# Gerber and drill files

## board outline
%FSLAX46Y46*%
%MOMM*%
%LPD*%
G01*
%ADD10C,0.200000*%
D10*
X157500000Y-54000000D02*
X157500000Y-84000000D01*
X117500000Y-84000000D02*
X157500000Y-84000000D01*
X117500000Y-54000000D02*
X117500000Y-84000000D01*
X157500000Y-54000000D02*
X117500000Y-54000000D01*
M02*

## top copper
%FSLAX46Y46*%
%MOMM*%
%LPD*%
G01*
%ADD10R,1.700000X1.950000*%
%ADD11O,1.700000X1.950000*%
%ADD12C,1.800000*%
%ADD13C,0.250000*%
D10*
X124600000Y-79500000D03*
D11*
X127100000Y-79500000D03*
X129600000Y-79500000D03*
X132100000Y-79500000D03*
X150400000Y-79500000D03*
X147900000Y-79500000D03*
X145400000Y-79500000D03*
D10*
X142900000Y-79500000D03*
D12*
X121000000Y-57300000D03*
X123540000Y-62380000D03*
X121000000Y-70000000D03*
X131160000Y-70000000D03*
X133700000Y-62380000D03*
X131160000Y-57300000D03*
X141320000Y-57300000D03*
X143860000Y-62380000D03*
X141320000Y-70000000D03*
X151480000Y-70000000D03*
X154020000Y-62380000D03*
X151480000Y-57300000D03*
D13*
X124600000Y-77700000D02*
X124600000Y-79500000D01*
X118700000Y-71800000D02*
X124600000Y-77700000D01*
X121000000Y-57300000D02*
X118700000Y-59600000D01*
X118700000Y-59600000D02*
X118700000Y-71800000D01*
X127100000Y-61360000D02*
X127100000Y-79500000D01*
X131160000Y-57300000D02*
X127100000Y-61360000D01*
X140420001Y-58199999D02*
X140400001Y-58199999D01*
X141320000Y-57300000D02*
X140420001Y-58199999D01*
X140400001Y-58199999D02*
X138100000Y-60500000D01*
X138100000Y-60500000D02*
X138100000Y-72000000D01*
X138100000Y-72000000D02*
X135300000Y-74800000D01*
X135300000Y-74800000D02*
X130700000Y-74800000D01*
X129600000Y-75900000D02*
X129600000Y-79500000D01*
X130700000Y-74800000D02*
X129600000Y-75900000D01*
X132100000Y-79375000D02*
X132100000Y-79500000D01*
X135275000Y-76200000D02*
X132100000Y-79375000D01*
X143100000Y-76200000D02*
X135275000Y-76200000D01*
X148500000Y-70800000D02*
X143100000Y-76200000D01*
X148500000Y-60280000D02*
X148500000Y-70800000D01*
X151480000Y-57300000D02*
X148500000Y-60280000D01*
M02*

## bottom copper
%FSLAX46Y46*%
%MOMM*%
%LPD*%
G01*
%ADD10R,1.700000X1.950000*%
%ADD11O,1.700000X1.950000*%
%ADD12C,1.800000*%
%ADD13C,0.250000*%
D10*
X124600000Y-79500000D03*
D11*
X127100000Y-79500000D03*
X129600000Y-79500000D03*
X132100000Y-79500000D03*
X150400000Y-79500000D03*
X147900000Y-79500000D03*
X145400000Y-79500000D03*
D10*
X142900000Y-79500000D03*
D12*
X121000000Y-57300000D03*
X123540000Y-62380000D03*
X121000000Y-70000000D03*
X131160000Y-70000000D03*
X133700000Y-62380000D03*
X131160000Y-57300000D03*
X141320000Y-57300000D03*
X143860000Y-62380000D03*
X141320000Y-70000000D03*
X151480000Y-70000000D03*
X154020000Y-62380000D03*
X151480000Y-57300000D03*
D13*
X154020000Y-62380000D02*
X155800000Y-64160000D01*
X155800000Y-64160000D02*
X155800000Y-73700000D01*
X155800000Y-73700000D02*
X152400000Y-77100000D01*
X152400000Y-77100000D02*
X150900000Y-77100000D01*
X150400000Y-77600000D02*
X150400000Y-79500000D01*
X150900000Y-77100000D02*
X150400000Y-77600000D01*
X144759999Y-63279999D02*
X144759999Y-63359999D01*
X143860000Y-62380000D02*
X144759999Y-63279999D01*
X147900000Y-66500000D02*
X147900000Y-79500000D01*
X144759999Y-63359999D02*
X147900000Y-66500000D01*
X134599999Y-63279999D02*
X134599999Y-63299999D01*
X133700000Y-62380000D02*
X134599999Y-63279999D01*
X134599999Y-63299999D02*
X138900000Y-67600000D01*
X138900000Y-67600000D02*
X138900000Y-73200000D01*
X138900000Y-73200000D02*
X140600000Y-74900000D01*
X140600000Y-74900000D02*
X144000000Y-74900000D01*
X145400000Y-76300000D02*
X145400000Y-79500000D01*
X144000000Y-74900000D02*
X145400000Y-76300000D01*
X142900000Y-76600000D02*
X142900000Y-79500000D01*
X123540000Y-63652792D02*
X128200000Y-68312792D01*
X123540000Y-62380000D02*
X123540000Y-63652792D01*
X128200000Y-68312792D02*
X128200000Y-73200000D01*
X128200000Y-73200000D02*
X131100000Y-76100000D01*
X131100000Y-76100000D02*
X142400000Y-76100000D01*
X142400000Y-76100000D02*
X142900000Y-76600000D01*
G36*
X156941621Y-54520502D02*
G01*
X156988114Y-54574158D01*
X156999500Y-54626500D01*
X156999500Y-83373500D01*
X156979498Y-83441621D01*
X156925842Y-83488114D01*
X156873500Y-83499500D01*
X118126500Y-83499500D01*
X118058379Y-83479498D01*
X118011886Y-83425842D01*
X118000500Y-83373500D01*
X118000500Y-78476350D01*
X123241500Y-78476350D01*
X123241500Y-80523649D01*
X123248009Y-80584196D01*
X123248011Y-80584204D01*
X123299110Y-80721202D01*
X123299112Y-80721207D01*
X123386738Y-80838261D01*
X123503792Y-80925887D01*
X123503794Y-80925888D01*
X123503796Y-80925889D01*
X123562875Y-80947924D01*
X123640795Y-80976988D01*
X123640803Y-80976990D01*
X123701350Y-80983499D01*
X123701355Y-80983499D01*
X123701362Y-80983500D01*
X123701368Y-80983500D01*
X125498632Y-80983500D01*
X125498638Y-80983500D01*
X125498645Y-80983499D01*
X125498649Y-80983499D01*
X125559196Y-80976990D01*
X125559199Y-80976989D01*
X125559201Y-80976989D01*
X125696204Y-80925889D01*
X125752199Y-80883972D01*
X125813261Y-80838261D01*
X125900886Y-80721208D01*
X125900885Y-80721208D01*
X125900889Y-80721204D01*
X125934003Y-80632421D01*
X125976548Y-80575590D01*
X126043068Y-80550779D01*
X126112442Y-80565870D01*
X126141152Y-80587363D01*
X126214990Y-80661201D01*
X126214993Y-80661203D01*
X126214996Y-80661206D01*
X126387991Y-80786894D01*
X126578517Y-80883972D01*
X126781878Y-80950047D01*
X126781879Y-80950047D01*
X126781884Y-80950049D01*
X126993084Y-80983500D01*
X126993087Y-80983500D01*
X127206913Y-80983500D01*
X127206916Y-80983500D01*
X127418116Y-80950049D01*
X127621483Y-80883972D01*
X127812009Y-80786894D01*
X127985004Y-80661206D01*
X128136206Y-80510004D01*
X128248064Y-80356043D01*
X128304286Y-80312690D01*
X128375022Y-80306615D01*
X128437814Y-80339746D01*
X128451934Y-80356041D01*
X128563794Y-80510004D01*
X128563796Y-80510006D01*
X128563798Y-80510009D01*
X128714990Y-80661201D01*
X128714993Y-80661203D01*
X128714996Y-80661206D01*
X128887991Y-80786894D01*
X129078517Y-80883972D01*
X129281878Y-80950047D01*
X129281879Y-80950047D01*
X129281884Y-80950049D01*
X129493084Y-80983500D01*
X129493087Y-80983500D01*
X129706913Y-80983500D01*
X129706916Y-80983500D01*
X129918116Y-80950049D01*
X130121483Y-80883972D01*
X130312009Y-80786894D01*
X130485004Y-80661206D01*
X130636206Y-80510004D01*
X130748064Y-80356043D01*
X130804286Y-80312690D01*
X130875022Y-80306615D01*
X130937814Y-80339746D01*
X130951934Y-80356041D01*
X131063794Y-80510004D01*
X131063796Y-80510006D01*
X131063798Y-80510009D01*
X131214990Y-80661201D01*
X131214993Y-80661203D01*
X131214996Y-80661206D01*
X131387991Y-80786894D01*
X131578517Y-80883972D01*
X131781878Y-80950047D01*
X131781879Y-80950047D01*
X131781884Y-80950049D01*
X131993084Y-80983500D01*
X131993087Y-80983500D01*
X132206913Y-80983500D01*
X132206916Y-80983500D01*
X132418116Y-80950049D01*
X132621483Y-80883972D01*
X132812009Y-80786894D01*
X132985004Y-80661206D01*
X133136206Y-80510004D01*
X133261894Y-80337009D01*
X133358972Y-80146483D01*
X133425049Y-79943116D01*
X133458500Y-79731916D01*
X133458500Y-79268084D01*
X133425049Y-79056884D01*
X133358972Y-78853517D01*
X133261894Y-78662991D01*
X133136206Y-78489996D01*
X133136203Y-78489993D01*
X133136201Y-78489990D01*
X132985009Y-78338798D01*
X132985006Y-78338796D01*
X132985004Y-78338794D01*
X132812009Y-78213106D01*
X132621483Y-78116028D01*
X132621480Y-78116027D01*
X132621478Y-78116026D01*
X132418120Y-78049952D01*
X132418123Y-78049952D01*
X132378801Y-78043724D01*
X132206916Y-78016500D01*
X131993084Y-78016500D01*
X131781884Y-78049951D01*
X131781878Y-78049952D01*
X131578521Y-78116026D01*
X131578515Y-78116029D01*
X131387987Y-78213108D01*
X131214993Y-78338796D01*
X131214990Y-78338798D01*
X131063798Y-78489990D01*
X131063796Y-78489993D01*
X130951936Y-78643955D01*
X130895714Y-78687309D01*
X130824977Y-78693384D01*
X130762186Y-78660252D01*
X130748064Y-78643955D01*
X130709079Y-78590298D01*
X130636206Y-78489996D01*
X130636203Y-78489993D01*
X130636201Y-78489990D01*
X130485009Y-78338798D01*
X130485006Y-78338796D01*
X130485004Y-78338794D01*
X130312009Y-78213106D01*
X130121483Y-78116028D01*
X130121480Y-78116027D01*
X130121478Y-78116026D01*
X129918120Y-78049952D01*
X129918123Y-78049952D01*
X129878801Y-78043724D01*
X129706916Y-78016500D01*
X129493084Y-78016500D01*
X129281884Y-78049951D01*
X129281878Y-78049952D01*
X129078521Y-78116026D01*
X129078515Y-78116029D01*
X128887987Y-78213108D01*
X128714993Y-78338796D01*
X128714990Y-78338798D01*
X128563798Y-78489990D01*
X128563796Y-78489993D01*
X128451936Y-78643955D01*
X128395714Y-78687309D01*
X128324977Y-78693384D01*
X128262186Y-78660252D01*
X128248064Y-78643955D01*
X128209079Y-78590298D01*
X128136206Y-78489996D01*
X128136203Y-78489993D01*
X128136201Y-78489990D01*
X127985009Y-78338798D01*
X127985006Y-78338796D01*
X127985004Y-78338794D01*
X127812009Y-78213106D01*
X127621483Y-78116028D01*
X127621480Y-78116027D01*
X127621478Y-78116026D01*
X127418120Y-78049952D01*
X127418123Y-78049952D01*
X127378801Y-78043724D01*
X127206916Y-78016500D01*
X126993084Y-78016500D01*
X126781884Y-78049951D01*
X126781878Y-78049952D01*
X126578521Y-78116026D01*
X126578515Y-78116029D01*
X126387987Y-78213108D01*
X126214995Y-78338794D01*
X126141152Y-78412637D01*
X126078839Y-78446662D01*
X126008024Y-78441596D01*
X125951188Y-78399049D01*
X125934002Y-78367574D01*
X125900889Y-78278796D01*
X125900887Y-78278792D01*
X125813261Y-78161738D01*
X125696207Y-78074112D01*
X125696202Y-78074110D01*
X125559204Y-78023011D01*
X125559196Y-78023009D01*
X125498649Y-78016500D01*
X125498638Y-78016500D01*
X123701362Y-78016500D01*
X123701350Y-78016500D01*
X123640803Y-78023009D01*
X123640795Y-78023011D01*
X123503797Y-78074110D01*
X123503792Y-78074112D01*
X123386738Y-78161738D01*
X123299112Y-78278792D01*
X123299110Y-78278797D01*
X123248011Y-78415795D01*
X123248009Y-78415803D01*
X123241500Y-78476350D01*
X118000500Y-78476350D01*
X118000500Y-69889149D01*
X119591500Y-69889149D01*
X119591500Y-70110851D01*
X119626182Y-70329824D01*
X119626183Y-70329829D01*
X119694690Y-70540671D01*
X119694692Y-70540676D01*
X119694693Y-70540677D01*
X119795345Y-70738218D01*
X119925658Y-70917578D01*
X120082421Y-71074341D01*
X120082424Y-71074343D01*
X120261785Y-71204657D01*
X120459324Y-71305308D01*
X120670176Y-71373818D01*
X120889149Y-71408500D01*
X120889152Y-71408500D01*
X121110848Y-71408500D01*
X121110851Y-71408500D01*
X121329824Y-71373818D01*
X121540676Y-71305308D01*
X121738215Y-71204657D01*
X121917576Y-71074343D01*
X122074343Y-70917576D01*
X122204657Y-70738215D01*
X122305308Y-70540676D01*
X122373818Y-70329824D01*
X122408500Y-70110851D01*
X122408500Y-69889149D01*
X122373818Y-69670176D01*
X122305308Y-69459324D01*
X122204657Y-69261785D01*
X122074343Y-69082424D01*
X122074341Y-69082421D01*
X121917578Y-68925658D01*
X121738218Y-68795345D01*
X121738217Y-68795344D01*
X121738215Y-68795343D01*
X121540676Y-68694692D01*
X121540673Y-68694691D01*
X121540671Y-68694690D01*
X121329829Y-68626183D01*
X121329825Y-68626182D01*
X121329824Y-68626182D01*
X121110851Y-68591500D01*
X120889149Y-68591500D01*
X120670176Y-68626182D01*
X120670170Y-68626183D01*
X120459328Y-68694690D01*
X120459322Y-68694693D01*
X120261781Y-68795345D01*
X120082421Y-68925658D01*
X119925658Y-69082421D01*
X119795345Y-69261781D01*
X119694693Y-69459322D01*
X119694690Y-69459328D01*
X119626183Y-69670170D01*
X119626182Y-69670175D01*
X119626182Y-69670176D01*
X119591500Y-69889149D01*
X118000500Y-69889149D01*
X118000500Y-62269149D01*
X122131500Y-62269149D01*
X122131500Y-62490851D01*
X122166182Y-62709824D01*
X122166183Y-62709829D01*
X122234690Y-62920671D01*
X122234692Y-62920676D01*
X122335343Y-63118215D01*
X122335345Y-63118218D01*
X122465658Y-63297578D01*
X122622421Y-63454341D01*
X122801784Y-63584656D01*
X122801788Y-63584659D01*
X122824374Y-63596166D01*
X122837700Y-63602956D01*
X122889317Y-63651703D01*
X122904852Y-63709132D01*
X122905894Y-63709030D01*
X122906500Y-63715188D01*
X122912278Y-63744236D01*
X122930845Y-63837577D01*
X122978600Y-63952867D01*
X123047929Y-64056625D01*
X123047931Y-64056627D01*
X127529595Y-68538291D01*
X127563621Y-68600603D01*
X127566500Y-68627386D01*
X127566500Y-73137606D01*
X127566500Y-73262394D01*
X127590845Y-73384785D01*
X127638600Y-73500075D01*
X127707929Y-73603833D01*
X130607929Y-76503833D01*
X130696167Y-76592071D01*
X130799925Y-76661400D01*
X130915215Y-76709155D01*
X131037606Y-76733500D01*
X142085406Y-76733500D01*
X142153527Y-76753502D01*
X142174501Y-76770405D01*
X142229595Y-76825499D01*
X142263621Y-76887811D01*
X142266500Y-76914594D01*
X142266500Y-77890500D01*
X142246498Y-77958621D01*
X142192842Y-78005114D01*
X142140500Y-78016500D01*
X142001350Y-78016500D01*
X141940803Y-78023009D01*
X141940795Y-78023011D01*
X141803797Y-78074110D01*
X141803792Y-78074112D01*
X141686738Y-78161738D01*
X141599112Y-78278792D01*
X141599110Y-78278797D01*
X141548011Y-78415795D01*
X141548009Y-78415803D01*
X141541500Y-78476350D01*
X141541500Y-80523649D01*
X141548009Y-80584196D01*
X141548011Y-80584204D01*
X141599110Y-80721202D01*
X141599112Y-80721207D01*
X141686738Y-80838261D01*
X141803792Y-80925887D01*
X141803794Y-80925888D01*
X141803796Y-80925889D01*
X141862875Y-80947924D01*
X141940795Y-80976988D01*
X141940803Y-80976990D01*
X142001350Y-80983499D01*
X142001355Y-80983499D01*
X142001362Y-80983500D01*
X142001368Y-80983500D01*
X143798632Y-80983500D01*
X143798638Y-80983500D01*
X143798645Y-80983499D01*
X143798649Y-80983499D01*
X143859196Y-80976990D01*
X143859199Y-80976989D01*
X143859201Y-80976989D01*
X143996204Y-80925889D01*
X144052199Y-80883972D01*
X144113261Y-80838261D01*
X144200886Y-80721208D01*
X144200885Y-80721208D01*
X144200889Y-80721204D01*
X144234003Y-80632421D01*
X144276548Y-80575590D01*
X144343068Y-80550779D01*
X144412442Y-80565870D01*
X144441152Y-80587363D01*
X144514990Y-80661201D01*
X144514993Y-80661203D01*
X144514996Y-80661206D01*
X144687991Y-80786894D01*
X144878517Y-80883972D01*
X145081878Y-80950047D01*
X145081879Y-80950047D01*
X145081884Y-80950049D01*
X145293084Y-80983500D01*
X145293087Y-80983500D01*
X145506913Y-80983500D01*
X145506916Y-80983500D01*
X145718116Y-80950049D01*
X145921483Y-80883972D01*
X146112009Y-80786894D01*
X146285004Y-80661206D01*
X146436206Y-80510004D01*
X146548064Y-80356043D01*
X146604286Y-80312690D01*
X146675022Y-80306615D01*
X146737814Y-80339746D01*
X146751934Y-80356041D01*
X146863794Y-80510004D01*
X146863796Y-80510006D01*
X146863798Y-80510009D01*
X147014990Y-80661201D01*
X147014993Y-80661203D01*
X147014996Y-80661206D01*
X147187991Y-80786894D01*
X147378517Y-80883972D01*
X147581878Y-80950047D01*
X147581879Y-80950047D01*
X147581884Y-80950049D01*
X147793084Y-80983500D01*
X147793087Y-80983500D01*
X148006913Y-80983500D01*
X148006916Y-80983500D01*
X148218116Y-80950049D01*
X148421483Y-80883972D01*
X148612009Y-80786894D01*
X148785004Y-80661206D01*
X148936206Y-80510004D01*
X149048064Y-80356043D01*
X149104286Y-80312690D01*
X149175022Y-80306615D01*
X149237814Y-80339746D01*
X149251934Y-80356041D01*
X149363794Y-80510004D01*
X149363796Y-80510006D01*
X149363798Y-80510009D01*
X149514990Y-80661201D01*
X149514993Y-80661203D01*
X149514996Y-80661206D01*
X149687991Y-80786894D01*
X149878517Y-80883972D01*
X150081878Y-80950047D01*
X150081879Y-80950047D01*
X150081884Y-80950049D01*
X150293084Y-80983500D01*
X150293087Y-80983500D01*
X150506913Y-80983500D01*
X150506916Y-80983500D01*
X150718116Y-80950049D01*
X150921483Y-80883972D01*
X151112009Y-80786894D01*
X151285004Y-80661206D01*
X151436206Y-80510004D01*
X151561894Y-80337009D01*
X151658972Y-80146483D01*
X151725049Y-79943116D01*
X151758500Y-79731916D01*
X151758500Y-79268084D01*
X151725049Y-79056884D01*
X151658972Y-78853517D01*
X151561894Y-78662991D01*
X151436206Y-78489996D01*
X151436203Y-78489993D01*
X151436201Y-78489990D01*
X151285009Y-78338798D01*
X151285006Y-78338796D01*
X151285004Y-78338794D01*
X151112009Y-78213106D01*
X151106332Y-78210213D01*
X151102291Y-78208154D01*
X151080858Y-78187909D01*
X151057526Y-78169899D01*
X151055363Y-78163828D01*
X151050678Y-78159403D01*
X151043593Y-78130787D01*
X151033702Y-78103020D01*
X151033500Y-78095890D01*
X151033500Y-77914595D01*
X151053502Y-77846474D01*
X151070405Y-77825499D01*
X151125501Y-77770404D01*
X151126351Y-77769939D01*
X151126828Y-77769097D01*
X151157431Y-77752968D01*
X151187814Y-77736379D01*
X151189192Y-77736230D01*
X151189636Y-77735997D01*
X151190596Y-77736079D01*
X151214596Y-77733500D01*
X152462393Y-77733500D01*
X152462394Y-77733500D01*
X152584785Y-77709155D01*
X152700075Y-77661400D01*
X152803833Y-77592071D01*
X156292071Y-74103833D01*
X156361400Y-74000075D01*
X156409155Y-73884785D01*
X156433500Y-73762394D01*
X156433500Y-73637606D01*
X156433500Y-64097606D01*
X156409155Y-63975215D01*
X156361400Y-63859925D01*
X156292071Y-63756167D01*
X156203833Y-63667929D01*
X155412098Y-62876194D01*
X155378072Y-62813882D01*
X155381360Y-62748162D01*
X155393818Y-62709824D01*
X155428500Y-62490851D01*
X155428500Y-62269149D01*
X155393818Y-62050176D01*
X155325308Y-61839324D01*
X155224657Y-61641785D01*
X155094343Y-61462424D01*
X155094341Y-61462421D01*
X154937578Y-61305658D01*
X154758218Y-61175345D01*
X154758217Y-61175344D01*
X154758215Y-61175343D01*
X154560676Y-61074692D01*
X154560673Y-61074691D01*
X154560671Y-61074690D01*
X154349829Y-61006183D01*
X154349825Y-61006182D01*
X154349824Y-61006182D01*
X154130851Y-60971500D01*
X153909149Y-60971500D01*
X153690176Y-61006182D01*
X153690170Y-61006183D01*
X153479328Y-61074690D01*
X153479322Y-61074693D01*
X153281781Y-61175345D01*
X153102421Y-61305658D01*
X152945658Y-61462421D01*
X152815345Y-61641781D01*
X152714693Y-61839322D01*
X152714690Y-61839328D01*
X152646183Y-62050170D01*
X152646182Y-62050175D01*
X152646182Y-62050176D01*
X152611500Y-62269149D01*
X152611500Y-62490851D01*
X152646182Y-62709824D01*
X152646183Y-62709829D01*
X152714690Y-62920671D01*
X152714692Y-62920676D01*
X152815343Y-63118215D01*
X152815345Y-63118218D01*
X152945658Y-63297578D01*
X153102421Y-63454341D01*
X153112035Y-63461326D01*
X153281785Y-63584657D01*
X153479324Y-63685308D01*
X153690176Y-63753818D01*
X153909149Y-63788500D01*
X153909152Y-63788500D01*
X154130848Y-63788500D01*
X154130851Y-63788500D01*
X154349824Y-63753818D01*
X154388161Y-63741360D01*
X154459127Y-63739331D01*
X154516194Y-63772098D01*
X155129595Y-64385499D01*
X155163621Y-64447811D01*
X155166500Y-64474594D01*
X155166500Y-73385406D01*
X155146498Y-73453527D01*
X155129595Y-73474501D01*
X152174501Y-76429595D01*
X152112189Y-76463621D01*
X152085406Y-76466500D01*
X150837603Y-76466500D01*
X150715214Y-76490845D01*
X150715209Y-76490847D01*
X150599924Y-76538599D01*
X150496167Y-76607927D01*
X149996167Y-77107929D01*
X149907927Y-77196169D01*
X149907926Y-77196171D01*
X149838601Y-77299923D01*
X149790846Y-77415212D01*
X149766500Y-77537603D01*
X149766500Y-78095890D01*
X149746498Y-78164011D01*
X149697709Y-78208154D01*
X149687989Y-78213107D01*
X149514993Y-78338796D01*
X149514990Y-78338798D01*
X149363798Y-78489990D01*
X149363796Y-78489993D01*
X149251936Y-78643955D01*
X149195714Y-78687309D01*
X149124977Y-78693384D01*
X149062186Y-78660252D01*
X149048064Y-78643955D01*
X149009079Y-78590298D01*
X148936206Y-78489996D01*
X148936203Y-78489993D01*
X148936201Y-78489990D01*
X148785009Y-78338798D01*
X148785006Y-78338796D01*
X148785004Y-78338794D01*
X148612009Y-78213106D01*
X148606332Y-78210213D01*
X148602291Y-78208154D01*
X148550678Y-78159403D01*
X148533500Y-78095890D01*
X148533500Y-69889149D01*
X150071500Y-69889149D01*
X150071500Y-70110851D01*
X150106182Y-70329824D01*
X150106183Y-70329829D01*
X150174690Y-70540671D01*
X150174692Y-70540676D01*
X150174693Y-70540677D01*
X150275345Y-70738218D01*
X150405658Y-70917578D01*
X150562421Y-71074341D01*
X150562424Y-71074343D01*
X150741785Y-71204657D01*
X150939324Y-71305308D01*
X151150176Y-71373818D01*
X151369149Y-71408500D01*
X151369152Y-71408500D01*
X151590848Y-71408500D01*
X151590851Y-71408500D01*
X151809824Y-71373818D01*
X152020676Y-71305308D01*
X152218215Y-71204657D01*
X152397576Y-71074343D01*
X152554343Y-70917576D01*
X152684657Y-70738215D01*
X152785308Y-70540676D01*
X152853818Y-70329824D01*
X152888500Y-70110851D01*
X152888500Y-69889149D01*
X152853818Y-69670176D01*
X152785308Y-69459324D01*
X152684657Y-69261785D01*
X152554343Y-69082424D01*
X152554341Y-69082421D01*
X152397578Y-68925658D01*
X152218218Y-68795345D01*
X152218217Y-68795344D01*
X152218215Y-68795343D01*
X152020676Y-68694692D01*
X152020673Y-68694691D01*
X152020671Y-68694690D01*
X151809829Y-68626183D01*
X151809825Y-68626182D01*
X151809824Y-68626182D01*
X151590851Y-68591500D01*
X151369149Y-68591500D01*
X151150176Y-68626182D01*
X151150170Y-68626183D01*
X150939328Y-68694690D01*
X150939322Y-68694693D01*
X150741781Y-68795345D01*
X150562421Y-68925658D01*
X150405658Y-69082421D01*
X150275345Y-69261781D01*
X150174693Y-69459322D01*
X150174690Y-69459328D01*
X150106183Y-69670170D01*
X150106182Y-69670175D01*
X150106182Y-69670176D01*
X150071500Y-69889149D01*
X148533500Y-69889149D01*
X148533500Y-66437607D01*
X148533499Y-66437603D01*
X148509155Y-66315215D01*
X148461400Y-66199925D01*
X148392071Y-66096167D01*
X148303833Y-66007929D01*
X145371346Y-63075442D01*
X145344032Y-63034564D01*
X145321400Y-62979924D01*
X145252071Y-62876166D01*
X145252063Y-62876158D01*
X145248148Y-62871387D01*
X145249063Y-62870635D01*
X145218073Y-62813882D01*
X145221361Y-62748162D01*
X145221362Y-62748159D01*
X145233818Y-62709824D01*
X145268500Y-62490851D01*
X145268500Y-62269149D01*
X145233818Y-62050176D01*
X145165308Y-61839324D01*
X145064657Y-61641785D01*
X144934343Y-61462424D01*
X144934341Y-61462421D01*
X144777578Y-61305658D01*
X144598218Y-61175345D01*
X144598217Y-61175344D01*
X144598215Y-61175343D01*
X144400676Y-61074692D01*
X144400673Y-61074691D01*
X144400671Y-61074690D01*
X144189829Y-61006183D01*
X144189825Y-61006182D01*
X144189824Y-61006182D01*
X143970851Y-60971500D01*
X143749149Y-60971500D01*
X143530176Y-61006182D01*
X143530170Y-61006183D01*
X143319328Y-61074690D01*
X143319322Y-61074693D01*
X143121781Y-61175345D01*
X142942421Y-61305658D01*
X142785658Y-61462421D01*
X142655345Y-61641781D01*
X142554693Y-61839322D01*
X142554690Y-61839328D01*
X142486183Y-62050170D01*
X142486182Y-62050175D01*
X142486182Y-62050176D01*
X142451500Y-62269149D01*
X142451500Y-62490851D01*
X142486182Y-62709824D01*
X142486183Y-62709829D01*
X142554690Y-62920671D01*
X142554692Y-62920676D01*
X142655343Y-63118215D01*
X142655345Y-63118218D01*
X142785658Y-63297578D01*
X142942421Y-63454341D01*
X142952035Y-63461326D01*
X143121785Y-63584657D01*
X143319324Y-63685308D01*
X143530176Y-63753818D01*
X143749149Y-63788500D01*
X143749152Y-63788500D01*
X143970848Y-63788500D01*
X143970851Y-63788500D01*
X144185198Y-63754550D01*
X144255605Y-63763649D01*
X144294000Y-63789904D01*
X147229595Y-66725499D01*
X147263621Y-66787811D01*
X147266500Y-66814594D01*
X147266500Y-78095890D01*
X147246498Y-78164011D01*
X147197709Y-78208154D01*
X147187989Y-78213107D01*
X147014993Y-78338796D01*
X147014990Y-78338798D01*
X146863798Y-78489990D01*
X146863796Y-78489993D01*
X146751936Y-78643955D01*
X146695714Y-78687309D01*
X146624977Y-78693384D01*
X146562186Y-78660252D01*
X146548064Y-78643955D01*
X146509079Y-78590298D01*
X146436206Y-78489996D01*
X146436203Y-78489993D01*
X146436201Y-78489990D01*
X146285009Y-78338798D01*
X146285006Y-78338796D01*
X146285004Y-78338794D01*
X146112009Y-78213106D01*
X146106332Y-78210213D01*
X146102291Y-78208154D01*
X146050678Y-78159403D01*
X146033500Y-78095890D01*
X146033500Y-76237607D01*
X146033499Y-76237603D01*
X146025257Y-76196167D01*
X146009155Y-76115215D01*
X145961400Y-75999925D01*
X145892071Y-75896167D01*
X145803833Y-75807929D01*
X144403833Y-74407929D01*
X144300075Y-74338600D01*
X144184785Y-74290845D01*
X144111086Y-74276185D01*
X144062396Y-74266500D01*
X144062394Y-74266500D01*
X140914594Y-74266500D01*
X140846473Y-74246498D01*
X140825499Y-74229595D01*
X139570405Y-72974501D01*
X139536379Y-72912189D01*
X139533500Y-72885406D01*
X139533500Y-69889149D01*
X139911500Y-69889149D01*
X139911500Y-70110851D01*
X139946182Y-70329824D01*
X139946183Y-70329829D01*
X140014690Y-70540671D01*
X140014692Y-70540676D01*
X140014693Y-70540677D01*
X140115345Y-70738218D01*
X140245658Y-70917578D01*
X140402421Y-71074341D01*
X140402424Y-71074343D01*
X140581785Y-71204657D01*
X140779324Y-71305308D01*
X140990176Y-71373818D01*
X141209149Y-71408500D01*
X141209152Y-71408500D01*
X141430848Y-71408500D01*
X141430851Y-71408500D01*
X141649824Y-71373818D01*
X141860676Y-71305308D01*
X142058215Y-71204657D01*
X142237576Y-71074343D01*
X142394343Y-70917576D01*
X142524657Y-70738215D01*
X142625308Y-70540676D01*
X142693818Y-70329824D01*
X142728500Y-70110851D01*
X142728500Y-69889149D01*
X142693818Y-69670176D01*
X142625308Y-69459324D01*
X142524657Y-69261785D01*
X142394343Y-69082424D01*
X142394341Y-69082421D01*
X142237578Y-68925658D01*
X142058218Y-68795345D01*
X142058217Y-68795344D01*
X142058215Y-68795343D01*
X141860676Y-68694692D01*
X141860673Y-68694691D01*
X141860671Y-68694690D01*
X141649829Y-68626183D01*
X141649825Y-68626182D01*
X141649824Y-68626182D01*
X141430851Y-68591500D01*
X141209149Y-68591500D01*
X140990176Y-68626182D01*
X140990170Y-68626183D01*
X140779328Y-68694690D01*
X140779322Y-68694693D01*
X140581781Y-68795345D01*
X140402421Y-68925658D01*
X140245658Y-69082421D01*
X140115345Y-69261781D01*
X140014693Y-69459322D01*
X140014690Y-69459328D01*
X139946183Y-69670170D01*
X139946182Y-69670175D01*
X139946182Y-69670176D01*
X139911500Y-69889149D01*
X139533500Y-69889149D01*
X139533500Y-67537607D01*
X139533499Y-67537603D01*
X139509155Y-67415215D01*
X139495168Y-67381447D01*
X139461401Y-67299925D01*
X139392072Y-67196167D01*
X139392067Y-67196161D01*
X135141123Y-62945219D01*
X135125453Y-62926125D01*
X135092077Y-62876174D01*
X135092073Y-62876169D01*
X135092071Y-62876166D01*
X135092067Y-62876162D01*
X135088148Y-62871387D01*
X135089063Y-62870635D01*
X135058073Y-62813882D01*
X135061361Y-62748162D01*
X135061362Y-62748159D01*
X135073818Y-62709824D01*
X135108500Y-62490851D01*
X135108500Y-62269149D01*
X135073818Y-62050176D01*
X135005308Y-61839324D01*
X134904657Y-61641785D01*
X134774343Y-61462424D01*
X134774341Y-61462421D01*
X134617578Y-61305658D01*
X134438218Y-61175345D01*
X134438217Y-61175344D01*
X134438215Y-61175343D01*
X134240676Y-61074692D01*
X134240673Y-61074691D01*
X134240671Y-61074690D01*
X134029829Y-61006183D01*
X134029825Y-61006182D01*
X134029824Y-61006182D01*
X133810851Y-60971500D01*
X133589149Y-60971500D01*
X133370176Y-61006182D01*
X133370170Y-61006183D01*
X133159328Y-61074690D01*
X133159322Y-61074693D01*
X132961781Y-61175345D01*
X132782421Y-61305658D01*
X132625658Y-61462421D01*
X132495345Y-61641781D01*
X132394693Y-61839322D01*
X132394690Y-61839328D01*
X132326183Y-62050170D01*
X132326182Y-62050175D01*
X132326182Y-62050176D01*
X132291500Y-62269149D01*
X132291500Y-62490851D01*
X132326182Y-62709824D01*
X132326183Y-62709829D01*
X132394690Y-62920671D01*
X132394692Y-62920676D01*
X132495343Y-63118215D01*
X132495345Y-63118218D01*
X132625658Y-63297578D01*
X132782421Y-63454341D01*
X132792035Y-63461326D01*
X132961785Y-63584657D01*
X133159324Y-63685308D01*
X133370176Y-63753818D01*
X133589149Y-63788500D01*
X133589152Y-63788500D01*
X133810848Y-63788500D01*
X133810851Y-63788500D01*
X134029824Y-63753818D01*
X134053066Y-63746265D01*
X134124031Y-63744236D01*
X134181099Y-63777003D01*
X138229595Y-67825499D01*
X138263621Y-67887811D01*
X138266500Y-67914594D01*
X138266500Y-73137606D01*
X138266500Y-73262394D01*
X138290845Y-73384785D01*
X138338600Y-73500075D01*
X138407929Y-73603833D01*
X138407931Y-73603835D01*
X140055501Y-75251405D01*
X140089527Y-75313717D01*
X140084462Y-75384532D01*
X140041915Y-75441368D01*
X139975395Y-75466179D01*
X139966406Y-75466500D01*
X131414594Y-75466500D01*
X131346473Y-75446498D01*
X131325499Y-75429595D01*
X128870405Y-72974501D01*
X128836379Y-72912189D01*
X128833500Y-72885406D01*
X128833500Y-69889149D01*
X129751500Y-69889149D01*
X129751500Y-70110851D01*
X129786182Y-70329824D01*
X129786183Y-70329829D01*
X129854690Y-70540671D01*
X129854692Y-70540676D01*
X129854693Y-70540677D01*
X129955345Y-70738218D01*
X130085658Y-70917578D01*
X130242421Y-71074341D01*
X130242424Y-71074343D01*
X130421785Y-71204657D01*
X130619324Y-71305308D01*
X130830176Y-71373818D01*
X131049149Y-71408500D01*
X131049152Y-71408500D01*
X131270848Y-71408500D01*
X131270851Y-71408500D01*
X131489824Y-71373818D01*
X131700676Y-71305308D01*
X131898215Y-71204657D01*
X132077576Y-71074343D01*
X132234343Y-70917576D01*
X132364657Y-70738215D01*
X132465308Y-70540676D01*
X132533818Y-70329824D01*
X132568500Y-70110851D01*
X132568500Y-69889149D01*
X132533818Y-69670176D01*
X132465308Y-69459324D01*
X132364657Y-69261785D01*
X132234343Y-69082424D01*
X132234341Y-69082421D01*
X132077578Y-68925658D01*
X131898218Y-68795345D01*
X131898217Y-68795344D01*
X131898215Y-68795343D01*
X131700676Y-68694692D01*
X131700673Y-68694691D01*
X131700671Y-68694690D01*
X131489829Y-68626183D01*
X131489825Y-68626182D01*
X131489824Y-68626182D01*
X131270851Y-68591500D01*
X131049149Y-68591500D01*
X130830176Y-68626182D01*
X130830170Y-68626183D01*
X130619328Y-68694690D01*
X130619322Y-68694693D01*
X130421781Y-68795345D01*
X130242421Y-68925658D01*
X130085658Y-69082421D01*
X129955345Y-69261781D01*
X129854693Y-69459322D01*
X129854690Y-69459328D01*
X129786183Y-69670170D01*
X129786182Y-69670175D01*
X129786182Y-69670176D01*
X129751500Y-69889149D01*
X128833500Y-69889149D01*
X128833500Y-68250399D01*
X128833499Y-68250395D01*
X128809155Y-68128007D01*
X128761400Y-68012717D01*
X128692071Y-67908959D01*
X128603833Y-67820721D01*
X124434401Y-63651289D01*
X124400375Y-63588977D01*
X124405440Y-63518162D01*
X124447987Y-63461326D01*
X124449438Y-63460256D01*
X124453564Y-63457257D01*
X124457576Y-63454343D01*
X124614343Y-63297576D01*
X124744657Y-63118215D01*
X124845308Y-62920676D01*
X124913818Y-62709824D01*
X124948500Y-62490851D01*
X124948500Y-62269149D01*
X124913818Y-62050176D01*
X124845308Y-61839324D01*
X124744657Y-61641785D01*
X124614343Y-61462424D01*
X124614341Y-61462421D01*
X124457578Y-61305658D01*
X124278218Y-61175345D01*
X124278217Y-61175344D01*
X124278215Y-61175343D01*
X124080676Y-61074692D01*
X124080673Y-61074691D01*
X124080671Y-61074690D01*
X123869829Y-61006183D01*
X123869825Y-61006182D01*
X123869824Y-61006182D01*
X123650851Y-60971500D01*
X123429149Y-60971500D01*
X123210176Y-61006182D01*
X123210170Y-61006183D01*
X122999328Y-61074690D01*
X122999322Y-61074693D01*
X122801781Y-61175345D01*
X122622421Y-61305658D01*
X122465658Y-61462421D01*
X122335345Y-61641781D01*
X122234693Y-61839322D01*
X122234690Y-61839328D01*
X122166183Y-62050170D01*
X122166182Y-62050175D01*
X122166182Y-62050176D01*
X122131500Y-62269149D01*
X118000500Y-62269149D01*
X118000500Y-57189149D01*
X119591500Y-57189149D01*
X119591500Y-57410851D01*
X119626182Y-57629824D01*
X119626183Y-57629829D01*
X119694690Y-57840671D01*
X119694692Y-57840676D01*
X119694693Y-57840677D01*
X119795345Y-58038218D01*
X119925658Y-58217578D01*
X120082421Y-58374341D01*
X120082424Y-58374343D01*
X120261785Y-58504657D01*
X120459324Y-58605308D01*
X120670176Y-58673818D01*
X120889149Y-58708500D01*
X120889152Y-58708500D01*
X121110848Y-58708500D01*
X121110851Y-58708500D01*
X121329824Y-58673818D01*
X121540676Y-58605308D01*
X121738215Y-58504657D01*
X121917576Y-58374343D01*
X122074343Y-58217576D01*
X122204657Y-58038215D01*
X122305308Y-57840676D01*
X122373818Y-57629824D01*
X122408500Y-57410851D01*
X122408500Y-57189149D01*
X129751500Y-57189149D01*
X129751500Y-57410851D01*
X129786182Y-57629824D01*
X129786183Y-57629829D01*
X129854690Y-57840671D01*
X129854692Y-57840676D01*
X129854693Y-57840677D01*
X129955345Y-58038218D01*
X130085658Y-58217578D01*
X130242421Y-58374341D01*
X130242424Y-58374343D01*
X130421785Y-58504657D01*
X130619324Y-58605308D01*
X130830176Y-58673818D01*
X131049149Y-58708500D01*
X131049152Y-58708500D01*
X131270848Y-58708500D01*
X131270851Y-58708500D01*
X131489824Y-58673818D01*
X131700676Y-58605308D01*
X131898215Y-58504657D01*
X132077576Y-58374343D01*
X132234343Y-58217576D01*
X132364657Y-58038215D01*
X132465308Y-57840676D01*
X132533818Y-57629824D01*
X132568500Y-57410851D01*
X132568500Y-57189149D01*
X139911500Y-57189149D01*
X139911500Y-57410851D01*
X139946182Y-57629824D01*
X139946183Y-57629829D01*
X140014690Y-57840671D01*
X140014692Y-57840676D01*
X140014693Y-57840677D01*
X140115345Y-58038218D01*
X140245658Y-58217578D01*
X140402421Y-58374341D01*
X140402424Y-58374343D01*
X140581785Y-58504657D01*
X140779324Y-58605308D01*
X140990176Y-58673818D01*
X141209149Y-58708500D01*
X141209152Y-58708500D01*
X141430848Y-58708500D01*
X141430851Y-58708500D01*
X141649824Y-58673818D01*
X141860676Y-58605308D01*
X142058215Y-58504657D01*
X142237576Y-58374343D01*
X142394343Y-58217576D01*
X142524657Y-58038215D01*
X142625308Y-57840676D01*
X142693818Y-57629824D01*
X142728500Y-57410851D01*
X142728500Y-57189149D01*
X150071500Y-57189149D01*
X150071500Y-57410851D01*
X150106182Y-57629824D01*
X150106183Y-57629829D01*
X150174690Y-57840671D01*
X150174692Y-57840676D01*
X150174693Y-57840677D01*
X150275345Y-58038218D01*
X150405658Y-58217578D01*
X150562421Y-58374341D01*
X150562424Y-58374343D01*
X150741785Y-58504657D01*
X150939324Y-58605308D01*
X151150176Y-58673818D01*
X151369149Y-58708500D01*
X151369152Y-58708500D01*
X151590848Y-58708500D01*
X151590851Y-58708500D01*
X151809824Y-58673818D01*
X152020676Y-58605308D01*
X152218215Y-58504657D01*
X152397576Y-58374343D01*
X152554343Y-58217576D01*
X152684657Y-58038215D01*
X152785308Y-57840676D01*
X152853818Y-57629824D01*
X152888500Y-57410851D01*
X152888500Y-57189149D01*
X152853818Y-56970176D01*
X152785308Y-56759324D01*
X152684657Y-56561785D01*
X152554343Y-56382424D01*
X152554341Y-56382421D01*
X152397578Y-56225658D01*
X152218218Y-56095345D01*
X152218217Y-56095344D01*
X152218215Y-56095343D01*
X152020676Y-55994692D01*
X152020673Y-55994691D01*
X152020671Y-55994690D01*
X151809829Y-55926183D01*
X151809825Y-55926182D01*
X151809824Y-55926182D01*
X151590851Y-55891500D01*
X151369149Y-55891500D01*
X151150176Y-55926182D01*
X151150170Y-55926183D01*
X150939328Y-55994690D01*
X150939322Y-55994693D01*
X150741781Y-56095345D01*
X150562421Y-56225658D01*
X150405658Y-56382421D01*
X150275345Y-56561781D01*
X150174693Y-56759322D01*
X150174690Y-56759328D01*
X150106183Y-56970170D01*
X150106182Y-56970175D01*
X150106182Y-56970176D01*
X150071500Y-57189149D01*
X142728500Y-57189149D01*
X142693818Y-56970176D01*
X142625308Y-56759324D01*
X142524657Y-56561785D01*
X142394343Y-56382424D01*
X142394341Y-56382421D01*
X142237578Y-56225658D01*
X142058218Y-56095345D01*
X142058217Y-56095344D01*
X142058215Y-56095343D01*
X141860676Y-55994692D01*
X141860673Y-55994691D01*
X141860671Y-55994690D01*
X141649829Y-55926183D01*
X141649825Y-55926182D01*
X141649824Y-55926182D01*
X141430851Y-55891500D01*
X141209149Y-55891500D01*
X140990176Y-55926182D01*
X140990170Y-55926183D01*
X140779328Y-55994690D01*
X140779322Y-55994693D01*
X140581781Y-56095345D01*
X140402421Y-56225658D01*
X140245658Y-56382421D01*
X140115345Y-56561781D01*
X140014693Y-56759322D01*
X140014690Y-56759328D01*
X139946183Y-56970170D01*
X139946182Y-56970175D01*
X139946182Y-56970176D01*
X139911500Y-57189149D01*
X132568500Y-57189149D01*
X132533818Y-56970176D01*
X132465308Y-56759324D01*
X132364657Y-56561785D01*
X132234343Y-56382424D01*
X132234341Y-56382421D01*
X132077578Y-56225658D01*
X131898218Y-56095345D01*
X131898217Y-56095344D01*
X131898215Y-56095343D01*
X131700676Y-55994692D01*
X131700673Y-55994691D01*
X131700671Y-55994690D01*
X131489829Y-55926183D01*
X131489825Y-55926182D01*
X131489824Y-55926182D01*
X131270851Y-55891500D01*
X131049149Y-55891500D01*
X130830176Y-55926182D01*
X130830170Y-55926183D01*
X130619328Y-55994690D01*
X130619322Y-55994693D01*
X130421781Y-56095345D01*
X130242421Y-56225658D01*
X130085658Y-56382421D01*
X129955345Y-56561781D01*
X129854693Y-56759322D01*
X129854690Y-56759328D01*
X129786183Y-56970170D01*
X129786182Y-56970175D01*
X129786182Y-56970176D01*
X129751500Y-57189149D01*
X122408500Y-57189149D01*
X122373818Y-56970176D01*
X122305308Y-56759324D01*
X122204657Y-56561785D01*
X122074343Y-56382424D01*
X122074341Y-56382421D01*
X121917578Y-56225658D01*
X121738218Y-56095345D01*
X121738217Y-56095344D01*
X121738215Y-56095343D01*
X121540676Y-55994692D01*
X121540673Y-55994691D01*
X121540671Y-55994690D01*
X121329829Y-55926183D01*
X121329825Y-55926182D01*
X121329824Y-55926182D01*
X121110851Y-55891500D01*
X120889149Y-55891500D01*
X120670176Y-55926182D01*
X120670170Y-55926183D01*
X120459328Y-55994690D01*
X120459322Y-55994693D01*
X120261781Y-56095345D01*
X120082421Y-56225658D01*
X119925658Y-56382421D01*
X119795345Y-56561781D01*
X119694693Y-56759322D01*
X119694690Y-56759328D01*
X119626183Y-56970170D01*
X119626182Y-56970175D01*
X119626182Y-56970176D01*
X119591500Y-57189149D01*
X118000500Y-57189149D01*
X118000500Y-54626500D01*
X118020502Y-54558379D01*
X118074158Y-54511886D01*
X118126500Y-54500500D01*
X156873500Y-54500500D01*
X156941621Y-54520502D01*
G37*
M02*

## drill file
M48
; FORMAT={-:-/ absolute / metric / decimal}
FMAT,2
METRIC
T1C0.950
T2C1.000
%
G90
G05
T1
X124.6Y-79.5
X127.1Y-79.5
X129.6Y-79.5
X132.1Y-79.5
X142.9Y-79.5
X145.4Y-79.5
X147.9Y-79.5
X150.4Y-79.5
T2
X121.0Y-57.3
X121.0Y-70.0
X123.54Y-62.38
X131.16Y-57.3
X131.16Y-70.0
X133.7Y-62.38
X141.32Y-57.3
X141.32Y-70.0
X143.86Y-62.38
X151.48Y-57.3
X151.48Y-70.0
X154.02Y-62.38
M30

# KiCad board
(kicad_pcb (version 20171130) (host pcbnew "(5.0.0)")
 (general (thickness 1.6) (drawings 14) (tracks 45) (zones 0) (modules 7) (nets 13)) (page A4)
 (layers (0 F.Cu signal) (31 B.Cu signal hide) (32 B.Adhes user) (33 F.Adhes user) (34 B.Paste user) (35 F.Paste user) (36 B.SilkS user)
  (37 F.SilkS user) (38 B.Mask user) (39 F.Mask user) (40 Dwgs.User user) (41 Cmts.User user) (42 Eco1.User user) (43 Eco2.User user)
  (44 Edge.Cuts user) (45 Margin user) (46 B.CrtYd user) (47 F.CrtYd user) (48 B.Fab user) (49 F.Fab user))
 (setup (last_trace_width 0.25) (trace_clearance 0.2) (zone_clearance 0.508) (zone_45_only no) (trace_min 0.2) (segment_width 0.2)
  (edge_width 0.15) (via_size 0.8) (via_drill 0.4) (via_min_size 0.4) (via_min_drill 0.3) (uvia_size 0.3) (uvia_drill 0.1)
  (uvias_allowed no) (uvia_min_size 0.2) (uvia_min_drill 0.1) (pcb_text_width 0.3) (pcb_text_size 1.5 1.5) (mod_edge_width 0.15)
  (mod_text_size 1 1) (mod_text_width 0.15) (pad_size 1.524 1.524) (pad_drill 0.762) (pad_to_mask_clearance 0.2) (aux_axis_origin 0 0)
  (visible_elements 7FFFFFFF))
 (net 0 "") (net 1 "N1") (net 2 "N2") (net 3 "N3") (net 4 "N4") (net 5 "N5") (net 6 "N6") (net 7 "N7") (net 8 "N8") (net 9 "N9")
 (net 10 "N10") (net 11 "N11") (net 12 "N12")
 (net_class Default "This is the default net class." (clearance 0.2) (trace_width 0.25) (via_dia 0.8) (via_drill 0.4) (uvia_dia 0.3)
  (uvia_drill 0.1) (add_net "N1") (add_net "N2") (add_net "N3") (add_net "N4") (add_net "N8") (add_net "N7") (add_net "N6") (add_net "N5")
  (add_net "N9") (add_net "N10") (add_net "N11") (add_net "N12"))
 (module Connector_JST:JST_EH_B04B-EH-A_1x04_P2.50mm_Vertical (layer F.Cu) (at 124.6 79.5)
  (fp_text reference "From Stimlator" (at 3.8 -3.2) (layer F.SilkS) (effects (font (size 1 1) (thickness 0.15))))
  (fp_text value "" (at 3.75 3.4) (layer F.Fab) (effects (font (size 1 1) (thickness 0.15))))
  (pad 1 thru_hole rect (at 0 0) (size 1.7 1.95) (drill 0.95) (layers *.Cu *.Mask) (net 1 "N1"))
  (pad 2 thru_hole oval (at 2.5 0) (size 1.7 1.95) (drill 0.95) (layers *.Cu *.Mask) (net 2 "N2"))
  (pad 3 thru_hole oval (at 5 0) (size 1.7 1.95) (drill 0.95) (layers *.Cu *.Mask) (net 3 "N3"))
  (pad 4 thru_hole oval (at 7.5 0) (size 1.7 1.95) (drill 0.95) (layers *.Cu *.Mask) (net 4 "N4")))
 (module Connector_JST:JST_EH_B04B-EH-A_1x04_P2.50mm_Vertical (layer F.Cu) (at 142.9 79.5)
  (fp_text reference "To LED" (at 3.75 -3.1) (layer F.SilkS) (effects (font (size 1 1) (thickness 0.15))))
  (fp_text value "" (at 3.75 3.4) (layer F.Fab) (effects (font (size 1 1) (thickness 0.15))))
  (pad 4 thru_hole oval (at 7.5 0) (size 1.7 1.95) (drill 0.95) (layers *.Cu *.Mask) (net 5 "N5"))
  (pad 3 thru_hole oval (at 5 0) (size 1.7 1.95) (drill 0.95) (layers *.Cu *.Mask) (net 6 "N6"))
  (pad 2 thru_hole oval (at 2.5 0) (size 1.7 1.95) (drill 0.95) (layers *.Cu *.Mask) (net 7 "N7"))
  (pad 1 thru_hole rect (at 0 0) (size 1.7 1.95) (drill 0.95) (layers *.Cu *.Mask) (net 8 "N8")))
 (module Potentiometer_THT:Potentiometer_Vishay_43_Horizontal (layer F.Cu) (at 121 70 270)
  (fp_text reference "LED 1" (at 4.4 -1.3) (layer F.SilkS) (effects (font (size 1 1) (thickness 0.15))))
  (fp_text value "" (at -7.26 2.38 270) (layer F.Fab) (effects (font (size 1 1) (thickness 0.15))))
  (pad 3 thru_hole circle (at -12.7 0 270) (size 1.8 1.8) (drill 1) (layers *.Cu *.Mask) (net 1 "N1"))
  (pad 2 thru_hole circle (at -7.62 -2.54 270) (size 1.8 1.8) (drill 1) (layers *.Cu *.Mask) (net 8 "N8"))
  (pad 1 thru_hole circle (at 0 0 270) (size 1.8 1.8) (drill 1) (layers *.Cu *.Mask) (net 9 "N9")))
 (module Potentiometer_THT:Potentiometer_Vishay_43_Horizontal (layer F.Cu) (at 131.16 70 270)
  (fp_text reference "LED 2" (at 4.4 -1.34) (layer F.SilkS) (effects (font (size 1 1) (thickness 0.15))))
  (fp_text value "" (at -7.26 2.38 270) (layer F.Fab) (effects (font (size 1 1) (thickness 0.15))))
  (pad 1 thru_hole circle (at 0 0 270) (size 1.8 1.8) (drill 1) (layers *.Cu *.Mask) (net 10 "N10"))
  (pad 2 thru_hole circle (at -7.62 -2.54 270) (size 1.8 1.8) (drill 1) (layers *.Cu *.Mask) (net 7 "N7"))
  (pad 3 thru_hole circle (at -12.7 0 270) (size 1.8 1.8) (drill 1) (layers *.Cu *.Mask) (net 2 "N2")))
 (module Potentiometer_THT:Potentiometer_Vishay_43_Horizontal (layer F.Cu) (at 141.32 70 270)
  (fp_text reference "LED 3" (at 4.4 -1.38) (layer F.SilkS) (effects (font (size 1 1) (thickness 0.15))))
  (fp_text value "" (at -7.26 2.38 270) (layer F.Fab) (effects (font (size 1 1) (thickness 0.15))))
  (pad 3 thru_hole circle (at -12.7 0 270) (size 1.8 1.8) (drill 1) (layers *.Cu *.Mask) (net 3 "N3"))
  (pad 2 thru_hole circle (at -7.62 -2.54 270) (size 1.8 1.8) (drill 1) (layers *.Cu *.Mask) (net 6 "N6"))
  (pad 1 thru_hole circle (at 0 0 270) (size 1.8 1.8) (drill 1) (layers *.Cu *.Mask) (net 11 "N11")))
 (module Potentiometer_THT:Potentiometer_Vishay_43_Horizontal (layer F.Cu) (at 151.48 70 270)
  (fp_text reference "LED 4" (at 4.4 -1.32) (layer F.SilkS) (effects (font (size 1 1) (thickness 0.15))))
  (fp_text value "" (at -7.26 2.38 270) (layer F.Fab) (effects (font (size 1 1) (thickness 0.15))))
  (pad 1 thru_hole circle (at 0 0 270) (size 1.8 1.8) (drill 1) (layers *.Cu *.Mask) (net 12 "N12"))
  (pad 2 thru_hole circle (at -7.62 -2.54 270) (size 1.8 1.8) (drill 1) (layers *.Cu *.Mask) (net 5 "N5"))
  (pad 3 thru_hole circle (at -12.7 0 270) (size 1.8 1.8) (drill 1) (layers *.Cu *.Mask) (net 4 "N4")))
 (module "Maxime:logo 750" (layer B.Cu) (at 137.5 75.1 180)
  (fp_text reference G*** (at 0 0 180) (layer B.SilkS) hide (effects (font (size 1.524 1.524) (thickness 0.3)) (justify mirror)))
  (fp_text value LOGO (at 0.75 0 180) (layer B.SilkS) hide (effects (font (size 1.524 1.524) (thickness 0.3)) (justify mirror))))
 (gr_line (start 157.5 54) (end 157.5 84) (layer Edge.Cuts) (width 0.2))
 (gr_line (start 117.5 84) (end 157.5 84) (layer Edge.Cuts) (width 0.2))
 (gr_line (start 117.5 54) (end 117.5 84) (layer Edge.Cuts) (width 0.2))
 (gr_line (start 157.5 54) (end 117.5 54) (layer Edge.Cuts) (width 0.2))
 (segment (start 124.6 77.7) (end 124.6 79.5) (width 0.25) (layer F.Cu) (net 1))
 (segment (start 118.7 71.8) (end 124.6 77.7) (width 0.25) (layer F.Cu) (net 1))
 (segment (start 121 57.3) (end 118.7 59.6) (width 0.25) (layer F.Cu) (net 1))
 (segment (start 118.7 59.6) (end 118.7 71.8) (width 0.25) (layer F.Cu) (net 1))
 (segment (start 127.1 61.36) (end 127.1 79.5) (width 0.25) (layer F.Cu) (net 2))
 (segment (start 131.16 57.3) (end 127.1 61.36) (width 0.25) (layer F.Cu) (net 2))
 (segment (start 140.420001 58.199999) (end 140.400001 58.199999) (width 0.25) (layer F.Cu) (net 3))
 (segment (start 141.32 57.3) (end 140.420001 58.199999) (width 0.25) (layer F.Cu) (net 3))
 (segment (start 140.400001 58.199999) (end 138.1 60.5) (width 0.25) (layer F.Cu) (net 3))
 (segment (start 138.1 60.5) (end 138.1 72) (width 0.25) (layer F.Cu) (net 3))
 (segment (start 138.1 72) (end 135.3 74.8) (width 0.25) (layer F.Cu) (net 3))
 (segment (start 135.3 74.8) (end 130.7 74.8) (width 0.25) (layer F.Cu) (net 3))
 (segment (start 129.6 75.9) (end 129.6 79.5) (width 0.25) (layer F.Cu) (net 3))
 (segment (start 130.7 74.8) (end 129.6 75.9) (width 0.25) (layer F.Cu) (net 3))
 (segment (start 132.1 79.375) (end 132.1 79.5) (width 0.25) (layer F.Cu) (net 4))
 (segment (start 135.275 76.2) (end 132.1 79.375) (width 0.25) (layer F.Cu) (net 4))
 (segment (start 143.1 76.2) (end 135.275 76.2) (width 0.25) (layer F.Cu) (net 4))
 (segment (start 148.5 70.8) (end 143.1 76.2) (width 0.25) (layer F.Cu) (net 4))
 (segment (start 148.5 60.28) (end 148.5 70.8) (width 0.25) (layer F.Cu) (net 4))
 (segment (start 151.48 57.3) (end 148.5 60.28) (width 0.25) (layer F.Cu) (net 4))
 (segment (start 154.02 62.38) (end 155.8 64.16) (width 0.25) (layer B.Cu) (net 5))
 (segment (start 155.8 64.16) (end 155.8 73.7) (width 0.25) (layer B.Cu) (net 5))
 (segment (start 155.8 73.7) (end 152.4 77.1) (width 0.25) (layer B.Cu) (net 5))
 (segment (start 152.4 77.1) (end 150.9 77.1) (width 0.25) (layer B.Cu) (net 5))
 (segment (start 150.4 77.6) (end 150.4 79.5) (width 0.25) (layer B.Cu) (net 5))
 (segment (start 150.9 77.1) (end 150.4 77.6) (width 0.25) (layer B.Cu) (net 5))
 (segment (start 144.759999 63.279999) (end 144.759999 63.359999) (width 0.25) (layer B.Cu) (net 6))
 (segment (start 143.86 62.38) (end 144.759999 63.279999) (width 0.25) (layer B.Cu) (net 6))
 (segment (start 147.9 66.5) (end 147.9 79.5) (width 0.25) (layer B.Cu) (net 6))
 (segment (start 144.759999 63.359999) (end 147.9 66.5) (width 0.25) (layer B.Cu) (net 6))
 (segment (start 134.599999 63.279999) (end 134.599999 63.299999) (width 0.25) (layer B.Cu) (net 7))
 (segment (start 133.7 62.38) (end 134.599999 63.279999) (width 0.25) (layer B.Cu) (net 7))
 (segment (start 134.599999 63.299999) (end 138.9 67.6) (width 0.25) (layer B.Cu) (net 7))
 (segment (start 138.9 67.6) (end 138.9 73.2) (width 0.25) (layer B.Cu) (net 7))
 (segment (start 138.9 73.2) (end 140.6 74.9) (width 0.25) (layer B.Cu) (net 7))
 (segment (start 140.6 74.9) (end 144 74.9) (width 0.25) (layer B.Cu) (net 7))
 (segment (start 145.4 76.3) (end 145.4 79.5) (width 0.25) (layer B.Cu) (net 7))
 (segment (start 144 74.9) (end 145.4 76.3) (width 0.25) (layer B.Cu) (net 7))
 (segment (start 142.9 76.6) (end 142.9 79.5) (width 0.25) (layer B.Cu) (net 8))
 (segment (start 123.54 63.652792) (end 128.2 68.312792) (width 0.25) (layer B.Cu) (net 8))
 (segment (start 123.54 62.38) (end 123.54 63.652792) (width 0.25) (layer B.Cu) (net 8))
 (segment (start 128.2 68.312792) (end 128.2 73.2) (width 0.25) (layer B.Cu) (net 8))
 (segment (start 128.2 73.2) (end 131.1 76.1) (width 0.25) (layer B.Cu) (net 8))
 (segment (start 131.1 76.1) (end 142.4 76.1) (width 0.25) (layer B.Cu) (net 8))
 (segment (start 142.4 76.1) (end 142.9 76.6) (width 0.25) (layer B.Cu) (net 8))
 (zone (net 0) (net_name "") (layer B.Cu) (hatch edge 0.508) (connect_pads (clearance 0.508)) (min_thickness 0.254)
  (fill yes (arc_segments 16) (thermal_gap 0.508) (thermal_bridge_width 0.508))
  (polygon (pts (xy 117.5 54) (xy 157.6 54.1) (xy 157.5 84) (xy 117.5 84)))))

